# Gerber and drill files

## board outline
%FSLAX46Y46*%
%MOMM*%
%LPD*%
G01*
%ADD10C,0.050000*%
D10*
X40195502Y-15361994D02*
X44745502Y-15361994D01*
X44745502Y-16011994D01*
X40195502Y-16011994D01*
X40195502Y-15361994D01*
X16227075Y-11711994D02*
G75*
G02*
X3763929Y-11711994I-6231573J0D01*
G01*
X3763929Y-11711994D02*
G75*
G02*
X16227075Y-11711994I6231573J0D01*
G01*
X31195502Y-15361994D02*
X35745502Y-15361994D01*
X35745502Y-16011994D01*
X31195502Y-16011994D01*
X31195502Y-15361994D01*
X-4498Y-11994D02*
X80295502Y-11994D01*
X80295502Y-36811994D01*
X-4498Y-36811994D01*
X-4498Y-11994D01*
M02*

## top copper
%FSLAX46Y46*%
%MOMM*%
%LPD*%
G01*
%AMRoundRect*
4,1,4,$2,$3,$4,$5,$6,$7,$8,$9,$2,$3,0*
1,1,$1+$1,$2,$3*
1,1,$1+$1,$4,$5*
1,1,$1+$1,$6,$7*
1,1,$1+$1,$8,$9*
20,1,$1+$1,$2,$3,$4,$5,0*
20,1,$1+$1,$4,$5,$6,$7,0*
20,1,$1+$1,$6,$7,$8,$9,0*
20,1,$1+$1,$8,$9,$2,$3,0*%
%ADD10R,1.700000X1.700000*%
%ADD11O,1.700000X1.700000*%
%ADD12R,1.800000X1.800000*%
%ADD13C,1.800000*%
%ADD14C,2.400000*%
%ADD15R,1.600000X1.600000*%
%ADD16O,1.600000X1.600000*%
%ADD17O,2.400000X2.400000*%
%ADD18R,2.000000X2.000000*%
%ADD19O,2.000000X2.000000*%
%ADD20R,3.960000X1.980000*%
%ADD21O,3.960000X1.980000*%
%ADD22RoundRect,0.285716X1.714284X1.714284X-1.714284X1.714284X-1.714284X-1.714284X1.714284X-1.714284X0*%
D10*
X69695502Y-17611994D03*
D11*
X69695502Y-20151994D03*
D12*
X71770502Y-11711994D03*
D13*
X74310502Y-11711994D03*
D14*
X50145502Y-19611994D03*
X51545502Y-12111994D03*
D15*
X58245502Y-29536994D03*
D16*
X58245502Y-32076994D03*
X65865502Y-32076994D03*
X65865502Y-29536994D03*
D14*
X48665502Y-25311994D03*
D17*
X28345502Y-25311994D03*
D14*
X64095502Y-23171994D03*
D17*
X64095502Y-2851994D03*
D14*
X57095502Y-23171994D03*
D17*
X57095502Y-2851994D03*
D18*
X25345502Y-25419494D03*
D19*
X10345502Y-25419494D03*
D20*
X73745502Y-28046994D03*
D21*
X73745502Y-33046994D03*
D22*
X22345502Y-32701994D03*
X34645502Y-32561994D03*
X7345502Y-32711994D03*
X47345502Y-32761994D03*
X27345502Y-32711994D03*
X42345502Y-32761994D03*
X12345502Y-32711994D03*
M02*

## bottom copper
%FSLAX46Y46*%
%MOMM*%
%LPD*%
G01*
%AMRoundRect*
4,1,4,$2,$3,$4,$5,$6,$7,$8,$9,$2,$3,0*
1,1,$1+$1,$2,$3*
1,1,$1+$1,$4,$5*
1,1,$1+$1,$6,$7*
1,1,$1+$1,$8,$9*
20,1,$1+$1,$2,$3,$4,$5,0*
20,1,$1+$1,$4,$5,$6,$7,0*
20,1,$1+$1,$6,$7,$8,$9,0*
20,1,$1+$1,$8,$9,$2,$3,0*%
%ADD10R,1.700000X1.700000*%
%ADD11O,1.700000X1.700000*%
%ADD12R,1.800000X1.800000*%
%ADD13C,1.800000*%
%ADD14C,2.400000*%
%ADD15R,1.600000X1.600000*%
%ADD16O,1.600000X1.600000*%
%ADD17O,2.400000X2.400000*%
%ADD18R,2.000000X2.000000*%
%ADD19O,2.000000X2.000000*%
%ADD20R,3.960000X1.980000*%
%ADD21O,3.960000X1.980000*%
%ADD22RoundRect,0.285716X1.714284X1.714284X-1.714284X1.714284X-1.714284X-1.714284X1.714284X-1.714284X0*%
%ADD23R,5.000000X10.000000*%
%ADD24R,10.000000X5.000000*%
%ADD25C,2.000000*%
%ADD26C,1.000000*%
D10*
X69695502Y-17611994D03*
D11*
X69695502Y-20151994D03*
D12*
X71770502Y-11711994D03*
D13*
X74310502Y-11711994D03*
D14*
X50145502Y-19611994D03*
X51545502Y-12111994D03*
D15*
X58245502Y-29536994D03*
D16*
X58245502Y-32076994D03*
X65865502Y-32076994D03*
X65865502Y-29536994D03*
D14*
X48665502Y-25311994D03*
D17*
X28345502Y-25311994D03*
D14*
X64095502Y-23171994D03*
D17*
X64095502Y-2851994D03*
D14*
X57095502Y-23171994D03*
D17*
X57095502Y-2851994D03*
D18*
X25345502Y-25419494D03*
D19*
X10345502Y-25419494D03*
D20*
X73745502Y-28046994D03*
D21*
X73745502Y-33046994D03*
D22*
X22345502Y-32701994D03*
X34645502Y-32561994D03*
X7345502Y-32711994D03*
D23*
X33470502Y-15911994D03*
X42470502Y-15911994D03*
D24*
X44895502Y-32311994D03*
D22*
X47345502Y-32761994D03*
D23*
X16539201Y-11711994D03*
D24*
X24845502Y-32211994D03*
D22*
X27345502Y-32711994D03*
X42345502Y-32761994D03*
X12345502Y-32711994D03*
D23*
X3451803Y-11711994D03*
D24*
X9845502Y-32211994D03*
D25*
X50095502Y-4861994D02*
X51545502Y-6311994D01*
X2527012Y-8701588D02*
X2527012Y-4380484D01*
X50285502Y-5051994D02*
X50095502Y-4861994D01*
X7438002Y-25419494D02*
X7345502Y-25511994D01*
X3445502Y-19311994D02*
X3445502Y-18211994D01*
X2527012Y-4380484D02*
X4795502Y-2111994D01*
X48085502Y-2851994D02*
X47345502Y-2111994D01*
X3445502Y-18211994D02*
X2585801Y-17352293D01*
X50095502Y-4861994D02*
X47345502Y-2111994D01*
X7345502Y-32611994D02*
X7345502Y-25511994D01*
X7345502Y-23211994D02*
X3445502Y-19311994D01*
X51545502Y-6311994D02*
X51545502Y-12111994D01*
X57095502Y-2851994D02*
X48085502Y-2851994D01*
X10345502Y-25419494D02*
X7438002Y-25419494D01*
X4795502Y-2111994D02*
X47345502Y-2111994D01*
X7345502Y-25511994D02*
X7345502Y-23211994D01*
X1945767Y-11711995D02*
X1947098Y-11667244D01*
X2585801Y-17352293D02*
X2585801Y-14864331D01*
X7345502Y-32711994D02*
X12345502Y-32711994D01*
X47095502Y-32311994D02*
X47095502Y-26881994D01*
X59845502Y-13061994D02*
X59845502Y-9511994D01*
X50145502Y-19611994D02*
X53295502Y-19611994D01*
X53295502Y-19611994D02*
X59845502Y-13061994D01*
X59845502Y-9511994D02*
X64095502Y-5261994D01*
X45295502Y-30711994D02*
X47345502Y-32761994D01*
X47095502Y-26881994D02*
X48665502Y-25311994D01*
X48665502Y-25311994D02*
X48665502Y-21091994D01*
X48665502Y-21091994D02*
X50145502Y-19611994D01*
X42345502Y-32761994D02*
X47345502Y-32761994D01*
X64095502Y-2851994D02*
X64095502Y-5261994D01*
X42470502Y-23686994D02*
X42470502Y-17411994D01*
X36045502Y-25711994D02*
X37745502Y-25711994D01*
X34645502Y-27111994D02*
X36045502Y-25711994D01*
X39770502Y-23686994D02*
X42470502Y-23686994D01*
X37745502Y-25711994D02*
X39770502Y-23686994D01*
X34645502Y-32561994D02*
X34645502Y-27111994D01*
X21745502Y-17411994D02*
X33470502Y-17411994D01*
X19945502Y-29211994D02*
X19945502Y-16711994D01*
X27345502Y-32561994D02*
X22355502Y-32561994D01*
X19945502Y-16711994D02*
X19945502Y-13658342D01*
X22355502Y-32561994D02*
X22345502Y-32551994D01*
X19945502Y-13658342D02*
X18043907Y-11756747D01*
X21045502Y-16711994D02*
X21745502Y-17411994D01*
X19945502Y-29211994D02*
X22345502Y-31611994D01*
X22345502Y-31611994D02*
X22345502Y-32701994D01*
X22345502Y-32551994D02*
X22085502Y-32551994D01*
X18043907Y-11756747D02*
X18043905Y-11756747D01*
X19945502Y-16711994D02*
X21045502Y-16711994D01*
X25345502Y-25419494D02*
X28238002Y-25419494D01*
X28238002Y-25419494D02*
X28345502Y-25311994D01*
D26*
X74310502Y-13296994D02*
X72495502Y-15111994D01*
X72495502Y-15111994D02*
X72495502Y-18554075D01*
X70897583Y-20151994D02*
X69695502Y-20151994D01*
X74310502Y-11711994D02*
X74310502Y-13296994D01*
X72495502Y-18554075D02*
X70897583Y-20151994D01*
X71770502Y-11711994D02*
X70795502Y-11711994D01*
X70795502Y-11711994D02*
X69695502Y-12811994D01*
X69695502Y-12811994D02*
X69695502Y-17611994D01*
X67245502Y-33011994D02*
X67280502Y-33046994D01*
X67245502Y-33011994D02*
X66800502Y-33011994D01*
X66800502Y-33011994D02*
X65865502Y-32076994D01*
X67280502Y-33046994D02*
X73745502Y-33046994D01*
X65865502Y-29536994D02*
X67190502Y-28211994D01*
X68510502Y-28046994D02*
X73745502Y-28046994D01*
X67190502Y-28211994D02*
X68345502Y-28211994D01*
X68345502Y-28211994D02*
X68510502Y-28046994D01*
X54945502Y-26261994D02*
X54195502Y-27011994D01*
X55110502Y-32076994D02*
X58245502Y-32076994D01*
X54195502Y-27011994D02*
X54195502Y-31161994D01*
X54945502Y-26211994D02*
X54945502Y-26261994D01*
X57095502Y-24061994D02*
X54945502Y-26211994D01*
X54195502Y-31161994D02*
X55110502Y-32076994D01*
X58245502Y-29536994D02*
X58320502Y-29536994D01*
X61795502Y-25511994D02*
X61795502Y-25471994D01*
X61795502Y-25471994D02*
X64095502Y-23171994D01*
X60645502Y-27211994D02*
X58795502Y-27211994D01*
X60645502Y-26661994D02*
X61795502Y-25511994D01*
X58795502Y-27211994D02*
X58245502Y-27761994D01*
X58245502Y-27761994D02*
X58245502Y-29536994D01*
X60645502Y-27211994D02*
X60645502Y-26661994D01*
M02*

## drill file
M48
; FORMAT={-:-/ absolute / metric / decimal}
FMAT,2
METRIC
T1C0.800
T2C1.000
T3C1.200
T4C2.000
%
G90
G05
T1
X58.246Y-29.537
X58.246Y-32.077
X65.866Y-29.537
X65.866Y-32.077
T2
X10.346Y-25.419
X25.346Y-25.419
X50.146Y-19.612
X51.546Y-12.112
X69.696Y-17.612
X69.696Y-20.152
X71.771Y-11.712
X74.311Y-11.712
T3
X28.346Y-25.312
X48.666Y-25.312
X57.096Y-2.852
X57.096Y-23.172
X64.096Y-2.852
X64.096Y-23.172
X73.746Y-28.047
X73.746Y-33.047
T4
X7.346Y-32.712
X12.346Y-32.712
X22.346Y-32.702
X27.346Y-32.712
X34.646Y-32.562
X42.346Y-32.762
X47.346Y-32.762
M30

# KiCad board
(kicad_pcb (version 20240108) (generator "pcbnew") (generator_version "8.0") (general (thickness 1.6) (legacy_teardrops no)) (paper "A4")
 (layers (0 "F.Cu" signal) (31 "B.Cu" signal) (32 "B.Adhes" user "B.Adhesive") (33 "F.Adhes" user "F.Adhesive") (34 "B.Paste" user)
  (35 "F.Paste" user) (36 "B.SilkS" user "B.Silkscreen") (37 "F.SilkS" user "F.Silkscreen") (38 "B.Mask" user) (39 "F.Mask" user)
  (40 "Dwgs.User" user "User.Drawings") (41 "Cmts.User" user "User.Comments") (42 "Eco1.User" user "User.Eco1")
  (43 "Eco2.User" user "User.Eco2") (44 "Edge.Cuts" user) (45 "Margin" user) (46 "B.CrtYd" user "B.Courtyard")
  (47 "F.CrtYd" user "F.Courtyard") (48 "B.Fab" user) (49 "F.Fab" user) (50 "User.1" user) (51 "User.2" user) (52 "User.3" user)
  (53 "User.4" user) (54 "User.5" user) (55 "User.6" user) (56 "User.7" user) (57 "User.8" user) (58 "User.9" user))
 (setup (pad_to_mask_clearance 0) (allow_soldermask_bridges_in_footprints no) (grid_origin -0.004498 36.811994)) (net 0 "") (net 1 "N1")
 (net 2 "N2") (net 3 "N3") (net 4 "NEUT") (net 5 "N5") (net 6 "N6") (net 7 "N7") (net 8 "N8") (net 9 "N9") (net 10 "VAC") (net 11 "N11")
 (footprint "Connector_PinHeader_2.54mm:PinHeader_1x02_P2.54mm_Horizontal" (layer "F.Cu") (at 69.695502 17.611994)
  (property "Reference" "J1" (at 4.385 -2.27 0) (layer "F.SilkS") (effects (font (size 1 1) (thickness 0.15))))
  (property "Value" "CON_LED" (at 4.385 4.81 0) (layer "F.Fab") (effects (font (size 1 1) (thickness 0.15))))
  (pad "1" thru_hole rect (at 0 0) (size 1.7 1.7) (drill 1) (layers "*.Cu" "*.Mask") (remove_unused_layers no) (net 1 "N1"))
  (pad "2" thru_hole oval (at 0 2.54) (size 1.7 1.7) (drill 1) (layers "*.Cu" "*.Mask") (remove_unused_layers no) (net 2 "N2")))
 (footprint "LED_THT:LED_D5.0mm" (layer "F.Cu") (at 71.770502 11.711994)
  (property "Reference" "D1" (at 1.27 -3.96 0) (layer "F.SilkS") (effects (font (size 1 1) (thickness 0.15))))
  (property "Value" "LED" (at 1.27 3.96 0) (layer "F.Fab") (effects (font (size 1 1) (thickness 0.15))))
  (pad "1" thru_hole rect (at 0 0) (size 1.8 1.8) (drill 1) (layers "*.Cu" "*.Mask") (remove_unused_layers no) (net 1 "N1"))
  (pad "2" thru_hole circle (at 2.54 0) (size 1.8 1.8) (drill 1) (layers "*.Cu" "*.Mask") (remove_unused_layers no) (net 2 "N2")))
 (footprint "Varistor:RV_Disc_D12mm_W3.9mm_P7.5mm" (layer "F.Cu") (at 50.145502 19.611994 90)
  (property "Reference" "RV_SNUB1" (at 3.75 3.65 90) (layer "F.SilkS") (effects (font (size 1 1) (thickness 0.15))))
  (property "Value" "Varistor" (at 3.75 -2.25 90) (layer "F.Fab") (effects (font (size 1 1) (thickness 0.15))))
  (pad "1" thru_hole circle (at 0 0 90) (size 2.4 2.4) (drill 1) (layers "*.Cu" "*.Mask") (remove_unused_layers no) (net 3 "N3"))
  (pad "2" thru_hole circle (at 7.5 1.4 90) (size 2.4 2.4) (drill 1) (layers "*.Cu" "*.Mask") (remove_unused_layers no) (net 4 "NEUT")))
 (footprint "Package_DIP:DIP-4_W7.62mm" (layer "F.Cu") (at 58.245502 29.536994)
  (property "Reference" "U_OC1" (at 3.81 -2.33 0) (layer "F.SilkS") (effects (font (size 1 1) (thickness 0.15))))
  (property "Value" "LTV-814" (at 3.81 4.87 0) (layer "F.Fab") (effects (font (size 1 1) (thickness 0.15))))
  (pad "1" thru_hole rect (at 0 0) (size 1.6 1.6) (drill 0.8) (layers "*.Cu" "*.Mask") (remove_unused_layers no) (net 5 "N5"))
  (pad "2" thru_hole oval (at 0 2.54) (size 1.6 1.6) (drill 0.8) (layers "*.Cu" "*.Mask") (remove_unused_layers no) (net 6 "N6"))
  (pad "3" thru_hole oval (at 7.62 2.54) (size 1.6 1.6) (drill 0.8) (layers "*.Cu" "*.Mask") (remove_unused_layers no) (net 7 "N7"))
  (pad "4" thru_hole oval (at 7.62 0) (size 1.6 1.6) (drill 0.8) (layers "*.Cu" "*.Mask") (remove_unused_layers no) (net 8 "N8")))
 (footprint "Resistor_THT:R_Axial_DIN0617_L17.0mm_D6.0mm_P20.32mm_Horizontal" (layer "F.Cu") (at 48.665502 25.311994 180)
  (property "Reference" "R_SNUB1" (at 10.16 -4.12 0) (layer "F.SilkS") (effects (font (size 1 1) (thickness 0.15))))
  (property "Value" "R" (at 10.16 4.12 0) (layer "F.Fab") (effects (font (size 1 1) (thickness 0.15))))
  (pad "1" thru_hole circle (at 0 0 180) (size 2.4 2.4) (drill 1.2) (layers "*.Cu" "*.Mask") (remove_unused_layers no) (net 3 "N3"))
  (pad "2" thru_hole oval (at 20.32 0 180) (size 2.4 2.4) (drill 1.2) (layers "*.Cu" "*.Mask") (remove_unused_layers no) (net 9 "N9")))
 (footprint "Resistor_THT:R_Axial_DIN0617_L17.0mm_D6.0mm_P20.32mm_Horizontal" (layer "F.Cu") (at 64.095502 23.171994 90)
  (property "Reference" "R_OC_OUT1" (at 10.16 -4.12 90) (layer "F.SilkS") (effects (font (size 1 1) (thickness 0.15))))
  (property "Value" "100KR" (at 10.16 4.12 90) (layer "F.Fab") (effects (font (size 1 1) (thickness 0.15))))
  (pad "1" thru_hole circle (at 0 0 90) (size 2.4 2.4) (drill 1.2) (layers "*.Cu" "*.Mask") (remove_unused_layers no) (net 5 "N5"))
  (pad "2" thru_hole oval (at 20.32 0 90) (size 2.4 2.4) (drill 1.2) (layers "*.Cu" "*.Mask") (remove_unused_layers no) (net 3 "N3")))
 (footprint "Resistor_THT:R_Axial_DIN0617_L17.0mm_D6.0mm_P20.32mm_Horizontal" (layer "F.Cu") (at 57.095502 23.171994 90)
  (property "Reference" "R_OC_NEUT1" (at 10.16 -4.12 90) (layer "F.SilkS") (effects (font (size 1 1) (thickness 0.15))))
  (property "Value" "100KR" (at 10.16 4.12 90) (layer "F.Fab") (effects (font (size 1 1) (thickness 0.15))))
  (pad "1" thru_hole circle (at 0 0 90) (size 2.4 2.4) (drill 1.2) (layers "*.Cu" "*.Mask") (remove_unused_layers no) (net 6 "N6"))
  (pad "2" thru_hole oval (at 20.32 0 90) (size 2.4 2.4) (drill 1.2) (layers "*.Cu" "*.Mask") (remove_unused_layers no) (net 4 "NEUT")))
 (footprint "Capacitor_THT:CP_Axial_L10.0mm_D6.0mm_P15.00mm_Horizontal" (layer "F.Cu") (at 25.345502 25.419494 180)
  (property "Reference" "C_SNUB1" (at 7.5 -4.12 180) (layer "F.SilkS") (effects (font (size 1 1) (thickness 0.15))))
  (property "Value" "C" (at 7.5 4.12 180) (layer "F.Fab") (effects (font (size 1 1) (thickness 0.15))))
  (pad "1" thru_hole rect (at 0 0 180) (size 2 2) (drill 1) (layers "*.Cu" "*.Mask") (remove_unused_layers no) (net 9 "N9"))
  (pad "2" thru_hole oval (at 15 0 180) (size 2 2) (drill 1) (layers "*.Cu" "*.Mask") (remove_unused_layers no) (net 4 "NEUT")))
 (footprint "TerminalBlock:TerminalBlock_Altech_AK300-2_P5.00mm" (layer "F.Cu") (at 73.745502 28.046994 -90)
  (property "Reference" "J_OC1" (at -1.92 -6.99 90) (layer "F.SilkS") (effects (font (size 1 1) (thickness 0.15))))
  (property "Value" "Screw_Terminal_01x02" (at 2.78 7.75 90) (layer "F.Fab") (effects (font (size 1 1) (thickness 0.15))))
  (pad "1" thru_hole rect (at 0 0 270) (size 1.98 3.96) (drill 1.2) (layers "*.Cu" "*.Mask") (remove_unused_layers no) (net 8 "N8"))
  (pad "2" thru_hole oval (at 5 0 270) (size 1.98 3.96) (drill 1.2) (layers "*.Cu" "*.Mask") (remove_unused_layers no) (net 7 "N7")))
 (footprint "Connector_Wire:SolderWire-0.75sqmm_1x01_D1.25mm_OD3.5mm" (layer "B.Cu") (at 22.345502 32.701994 180)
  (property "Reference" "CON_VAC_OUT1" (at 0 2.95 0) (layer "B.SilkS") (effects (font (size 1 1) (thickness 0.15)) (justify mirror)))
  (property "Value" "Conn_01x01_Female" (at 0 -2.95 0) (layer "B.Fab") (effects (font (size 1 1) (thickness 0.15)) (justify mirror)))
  (pad "1" thru_hole roundrect (at 0 0 180) (size 4 4) (drill 2) (layers "*.Cu" "*.Mask") (remove_unused_layers no)
   (roundrect_rratio 0.071429) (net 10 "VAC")))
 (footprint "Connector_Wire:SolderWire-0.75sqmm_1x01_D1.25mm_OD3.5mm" (layer "B.Cu") (at 34.645502 32.561994 180)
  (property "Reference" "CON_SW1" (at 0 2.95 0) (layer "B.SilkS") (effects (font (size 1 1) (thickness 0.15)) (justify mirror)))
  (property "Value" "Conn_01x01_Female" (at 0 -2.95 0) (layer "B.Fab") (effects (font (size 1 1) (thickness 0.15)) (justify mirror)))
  (pad "1" thru_hole roundrect (at 0 0 180) (size 4 4) (drill 2) (layers "*.Cu" "*.Mask") (remove_unused_layers no)
   (roundrect_rratio 0.071429) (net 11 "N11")))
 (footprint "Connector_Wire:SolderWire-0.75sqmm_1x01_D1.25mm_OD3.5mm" (layer "B.Cu") (at 7.345502 32.711994 180)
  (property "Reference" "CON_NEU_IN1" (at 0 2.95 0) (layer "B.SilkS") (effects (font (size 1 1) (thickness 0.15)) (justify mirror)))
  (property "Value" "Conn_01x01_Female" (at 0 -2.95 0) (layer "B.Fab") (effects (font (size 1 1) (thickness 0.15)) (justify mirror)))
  (pad "1" thru_hole roundrect (at 0 0 180) (size 4 4) (drill 2) (layers "*.Cu" "*.Mask") (remove_unused_layers no)
   (roundrect_rratio 0.071429) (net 4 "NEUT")))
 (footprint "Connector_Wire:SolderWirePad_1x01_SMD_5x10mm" (layer "B.Cu") (at 33.470502 15.911994 180)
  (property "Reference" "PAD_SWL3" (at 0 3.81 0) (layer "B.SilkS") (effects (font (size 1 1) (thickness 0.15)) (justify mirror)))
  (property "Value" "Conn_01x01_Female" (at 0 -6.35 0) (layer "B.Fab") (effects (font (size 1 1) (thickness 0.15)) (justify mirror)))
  (pad "1" smd rect (at 0 0 180) (size 5 10) (layers "B.Cu" "B.Paste" "B.Mask") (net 10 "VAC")))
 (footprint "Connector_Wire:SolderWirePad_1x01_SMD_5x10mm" (layer "B.Cu") (at 42.470502 15.911994 180)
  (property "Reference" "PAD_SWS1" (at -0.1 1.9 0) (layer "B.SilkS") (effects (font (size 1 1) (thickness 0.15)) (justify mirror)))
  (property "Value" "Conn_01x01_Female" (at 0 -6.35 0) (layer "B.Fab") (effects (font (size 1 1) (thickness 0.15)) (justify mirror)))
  (pad "1" smd rect (at 0 0 180) (size 5 10) (layers "B.Cu" "B.Paste" "B.Mask") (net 11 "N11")))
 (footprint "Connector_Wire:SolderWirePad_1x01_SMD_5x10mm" (layer "B.Cu") (at 44.895502 32.311994 -90)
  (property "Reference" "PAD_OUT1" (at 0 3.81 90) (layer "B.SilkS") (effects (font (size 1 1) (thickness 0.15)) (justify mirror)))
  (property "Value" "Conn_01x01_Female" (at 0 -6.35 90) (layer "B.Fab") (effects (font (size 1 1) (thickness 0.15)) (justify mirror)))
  (pad "1" smd rect (at 0 0 270) (size 5 10) (layers "B.Cu" "B.Paste" "B.Mask") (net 3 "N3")))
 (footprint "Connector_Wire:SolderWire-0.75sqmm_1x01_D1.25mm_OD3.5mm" (layer "B.Cu") (at 47.345502 32.761994 180)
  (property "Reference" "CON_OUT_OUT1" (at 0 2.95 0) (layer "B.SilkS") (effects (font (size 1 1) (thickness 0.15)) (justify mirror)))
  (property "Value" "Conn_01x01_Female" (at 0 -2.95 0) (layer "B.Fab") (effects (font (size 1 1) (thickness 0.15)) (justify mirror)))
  (pad "1" thru_hole roundrect (at 0 0 180) (size 4 4) (drill 2) (layers "*.Cu" "*.Mask") (remove_unused_layers no)
   (roundrect_rratio 0.071429) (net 3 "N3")))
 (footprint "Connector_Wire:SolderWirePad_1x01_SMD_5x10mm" (layer "B.Cu") (at 16.539201 11.711994 180)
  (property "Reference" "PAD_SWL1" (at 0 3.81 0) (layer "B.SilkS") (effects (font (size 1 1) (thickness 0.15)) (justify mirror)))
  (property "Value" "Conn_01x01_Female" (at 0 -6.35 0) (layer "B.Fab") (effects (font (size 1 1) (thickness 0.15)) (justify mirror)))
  (pad "1" smd rect (at 0 0 180) (size 5 10) (layers "B.Cu" "B.Paste" "B.Mask") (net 10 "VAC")))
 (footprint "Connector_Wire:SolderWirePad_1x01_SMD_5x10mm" (layer "B.Cu") (at 24.845502 32.211994 -90)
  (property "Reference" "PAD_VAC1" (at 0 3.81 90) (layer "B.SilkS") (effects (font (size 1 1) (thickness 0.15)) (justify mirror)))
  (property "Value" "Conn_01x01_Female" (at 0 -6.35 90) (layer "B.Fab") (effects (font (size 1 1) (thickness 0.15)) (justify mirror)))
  (pad "1" smd rect (at 0 0 270) (size 5 10) (layers "B.Cu" "B.Paste" "B.Mask") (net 10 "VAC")))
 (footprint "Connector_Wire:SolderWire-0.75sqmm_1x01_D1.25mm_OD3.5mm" (layer "B.Cu") (at 27.345502 32.711994 180)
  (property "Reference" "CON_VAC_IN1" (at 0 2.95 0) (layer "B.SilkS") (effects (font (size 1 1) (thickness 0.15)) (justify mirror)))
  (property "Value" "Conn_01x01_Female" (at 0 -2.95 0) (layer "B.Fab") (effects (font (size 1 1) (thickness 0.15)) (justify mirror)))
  (pad "1" thru_hole roundrect (at 0 0 180) (size 4 4) (drill 2) (layers "*.Cu" "*.Mask") (remove_unused_layers no)
   (roundrect_rratio 0.071429) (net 10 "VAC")))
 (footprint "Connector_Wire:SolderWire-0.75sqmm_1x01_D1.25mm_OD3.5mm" (layer "B.Cu") (at 42.345502 32.761994 180)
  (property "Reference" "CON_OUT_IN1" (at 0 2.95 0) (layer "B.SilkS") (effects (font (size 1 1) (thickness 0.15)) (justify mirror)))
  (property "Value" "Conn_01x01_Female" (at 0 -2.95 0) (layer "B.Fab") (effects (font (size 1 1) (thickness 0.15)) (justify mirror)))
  (pad "1" thru_hole roundrect (at 0 0 180) (size 4 4) (drill 2) (layers "*.Cu" "*.Mask") (remove_unused_layers no)
   (roundrect_rratio 0.071429) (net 3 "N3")))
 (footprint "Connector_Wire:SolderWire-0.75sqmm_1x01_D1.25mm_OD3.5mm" (layer "B.Cu") (at 12.345502 32.711994 180)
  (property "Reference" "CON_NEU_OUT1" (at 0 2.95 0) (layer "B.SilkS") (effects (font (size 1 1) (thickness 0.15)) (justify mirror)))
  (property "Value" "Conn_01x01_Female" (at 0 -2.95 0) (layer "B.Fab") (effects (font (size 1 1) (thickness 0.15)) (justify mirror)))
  (pad "1" thru_hole roundrect (at 0 0 180) (size 4 4) (drill 2) (layers "*.Cu" "*.Mask") (remove_unused_layers no)
   (roundrect_rratio 0.071429) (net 4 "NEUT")))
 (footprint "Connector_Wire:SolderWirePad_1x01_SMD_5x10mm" (layer "B.Cu") (at 3.451803 11.711994 180)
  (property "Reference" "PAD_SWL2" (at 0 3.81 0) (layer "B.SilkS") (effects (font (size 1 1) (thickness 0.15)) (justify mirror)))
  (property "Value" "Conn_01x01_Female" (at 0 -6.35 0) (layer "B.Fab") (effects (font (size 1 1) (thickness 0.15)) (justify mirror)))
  (pad "1" smd rect (at 0 0 180) (size 5 10) (layers "B.Cu" "B.Paste" "B.Mask") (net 4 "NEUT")))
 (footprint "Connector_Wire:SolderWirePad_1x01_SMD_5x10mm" (layer "B.Cu") (at 9.845502 32.211994 -90)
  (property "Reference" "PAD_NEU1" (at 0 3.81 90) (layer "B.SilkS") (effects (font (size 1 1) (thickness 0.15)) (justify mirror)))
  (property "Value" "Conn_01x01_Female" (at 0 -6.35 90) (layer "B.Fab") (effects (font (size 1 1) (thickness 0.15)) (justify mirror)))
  (pad "1" smd rect (at 0 0 270) (size 5 10) (layers "B.Cu" "B.Paste" "B.Mask") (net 4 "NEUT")))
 (gr_rect (start 40.195502 15.361994) (end 44.745502 16.011994) (stroke (width 0.05) (type default)) (fill none) (layer "Edge.Cuts"))
 (gr_circle (center 9.995502 11.711994) (end 13.845502 16.611994) (stroke (width 0.05) (type default)) (fill none) (layer "Edge.Cuts"))
 (gr_rect (start 31.195502 15.361994) (end 35.745502 16.011994) (stroke (width 0.05) (type default)) (fill none) (layer "Edge.Cuts"))
 (gr_rect (start -0.004498 0.011994) (end 80.295502 36.811994) (stroke (width 0.05) (type default)) (fill none) (layer "Edge.Cuts"))
 (segment (start 50.095502 4.861994) (end 51.545502 6.311994) (width 2) (layer "B.Cu") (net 4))
 (segment (start 2.527012 8.701588) (end 2.527012 4.380484) (width 2) (layer "B.Cu") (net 4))
 (segment (start 50.285502 5.051994) (end 50.095502 4.861994) (width 2) (layer "B.Cu") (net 4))
 (segment (start 7.438002 25.419494) (end 7.345502 25.511994) (width 2) (layer "B.Cu") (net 4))
 (segment (start 3.445502 19.311994) (end 3.445502 18.211994) (width 2) (layer "B.Cu") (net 4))
 (segment (start 2.527012 4.380484) (end 4.795502 2.111994) (width 2) (layer "B.Cu") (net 4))
 (segment (start 48.085502 2.851994) (end 47.345502 2.111994) (width 2) (layer "B.Cu") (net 4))
 (segment (start 3.445502 18.211994) (end 2.585801 17.352293) (width 2) (layer "B.Cu") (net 4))
 (segment (start 50.095502 4.861994) (end 47.345502 2.111994) (width 2) (layer "B.Cu") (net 4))
 (segment (start 7.345502 32.611994) (end 7.345502 25.511994) (width 2) (layer "B.Cu") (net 4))
 (segment (start 7.345502 23.211994) (end 3.445502 19.311994) (width 2) (layer "B.Cu") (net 4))
 (segment (start 51.545502 6.311994) (end 51.545502 12.111994) (width 2) (layer "B.Cu") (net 4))
 (segment (start 57.095502 2.851994) (end 48.085502 2.851994) (width 2) (layer "B.Cu") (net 4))
 (segment (start 10.345502 25.419494) (end 7.438002 25.419494) (width 2) (layer "B.Cu") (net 4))
 (segment (start 4.795502 2.111994) (end 47.345502 2.111994) (width 2) (layer "B.Cu") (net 4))
 (segment (start 7.345502 25.511994) (end 7.345502 23.211994) (width 2) (layer "B.Cu") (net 4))
 (segment (start 1.945767 11.711995) (end 1.947098 11.667244) (width 2) (layer "B.Cu") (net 4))
 (segment (start 2.585801 17.352293) (end 2.585801 14.864331) (width 2) (layer "B.Cu") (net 4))
 (segment (start 7.345502 32.711994) (end 12.345502 32.711994) (width 2) (layer "B.Cu") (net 4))
 (segment (start 47.095502 32.311994) (end 47.095502 26.881994) (width 2) (layer "B.Cu") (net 3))
 (segment (start 59.845502 13.061994) (end 59.845502 9.511994) (width 2) (layer "B.Cu") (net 3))
 (segment (start 50.145502 19.611994) (end 53.295502 19.611994) (width 2) (layer "B.Cu") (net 3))
 (segment (start 53.295502 19.611994) (end 59.845502 13.061994) (width 2) (layer "B.Cu") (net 3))
 (segment (start 59.845502 9.511994) (end 64.095502 5.261994) (width 2) (layer "B.Cu") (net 3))
 (segment (start 45.295502 30.711994) (end 47.345502 32.761994) (width 2) (layer "B.Cu") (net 3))
 (segment (start 47.095502 26.881994) (end 48.665502 25.311994) (width 2) (layer "B.Cu") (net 3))
 (segment (start 48.665502 25.311994) (end 48.665502 21.091994) (width 2) (layer "B.Cu") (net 3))
 (segment (start 48.665502 21.091994) (end 50.145502 19.611994) (width 2) (layer "B.Cu") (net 3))
 (segment (start 42.345502 32.761994) (end 47.345502 32.761994) (width 2) (layer "B.Cu") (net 3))
 (segment (start 64.095502 2.851994) (end 64.095502 5.261994) (width 2) (layer "B.Cu") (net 3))
 (segment (start 42.470502 23.686994) (end 42.470502 17.411994) (width 2) (layer "B.Cu") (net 11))
 (segment (start 36.045502 25.711994) (end 37.745502 25.711994) (width 2) (layer "B.Cu") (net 11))
 (segment (start 34.645502 27.111994) (end 36.045502 25.711994) (width 2) (layer "B.Cu") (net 11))
 (segment (start 39.770502 23.686994) (end 42.470502 23.686994) (width 2) (layer "B.Cu") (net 11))
 (segment (start 37.745502 25.711994) (end 39.770502 23.686994) (width 2) (layer "B.Cu") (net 11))
 (segment (start 34.645502 32.561994) (end 34.645502 27.111994) (width 2) (layer "B.Cu") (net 11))
 (segment (start 21.745502 17.411994) (end 33.470502 17.411994) (width 2) (layer "B.Cu") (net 10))
 (segment (start 19.945502 29.211994) (end 19.945502 16.711994) (width 2) (layer "B.Cu") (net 10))
 (segment (start 27.345502 32.561994) (end 22.355502 32.561994) (width 2) (layer "B.Cu") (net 10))
 (segment (start 19.945502 16.711994) (end 19.945502 13.658342) (width 2) (layer "B.Cu") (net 10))
 (segment (start 22.355502 32.561994) (end 22.345502 32.551994) (width 2) (layer "B.Cu") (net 10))
 (segment (start 19.945502 13.658342) (end 18.043907 11.756747) (width 2) (layer "B.Cu") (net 10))
 (segment (start 21.045502 16.711994) (end 21.745502 17.411994) (width 2) (layer "B.Cu") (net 10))
 (segment (start 19.945502 29.211994) (end 22.345502 31.611994) (width 2) (layer "B.Cu") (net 10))
 (segment (start 22.345502 31.611994) (end 22.345502 32.701994) (width 2) (layer "B.Cu") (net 10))
 (segment (start 22.345502 32.551994) (end 22.085502 32.551994) (width 2) (layer "B.Cu") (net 10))
 (segment (start 18.043907 11.756747) (end 18.043905 11.756747) (width 2) (layer "B.Cu") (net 10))
 (segment (start 19.945502 16.711994) (end 21.045502 16.711994) (width 2) (layer "B.Cu") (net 10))
 (segment (start 25.345502 25.419494) (end 28.238002 25.419494) (width 2) (layer "B.Cu") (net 9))
 (segment (start 28.238002 25.419494) (end 28.345502 25.311994) (width 2) (layer "B.Cu") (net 9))
 (segment (start 74.310502 13.296994) (end 72.495502 15.111994) (width 1) (layer "B.Cu") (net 2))
 (segment (start 72.495502 15.111994) (end 72.495502 18.554075) (width 1) (layer "B.Cu") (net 2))
 (segment (start 70.897583 20.151994) (end 69.695502 20.151994) (width 1) (layer "B.Cu") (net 2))
 (segment (start 74.310502 11.711994) (end 74.310502 13.296994) (width 1) (layer "B.Cu") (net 2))
 (segment (start 72.495502 18.554075) (end 70.897583 20.151994) (width 1) (layer "B.Cu") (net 2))
 (segment (start 71.770502 11.711994) (end 70.795502 11.711994) (width 1) (layer "B.Cu") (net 1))
 (segment (start 70.795502 11.711994) (end 69.695502 12.811994) (width 1) (layer "B.Cu") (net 1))
 (segment (start 69.695502 12.811994) (end 69.695502 17.611994) (width 1) (layer "B.Cu") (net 1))
 (segment (start 67.245502 33.011994) (end 67.280502 33.046994) (width 1) (layer "B.Cu") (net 7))
 (segment (start 67.245502 33.011994) (end 66.800502 33.011994) (width 1) (layer "B.Cu") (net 7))
 (segment (start 66.800502 33.011994) (end 65.865502 32.076994) (width 1) (layer "B.Cu") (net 7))
 (segment (start 67.280502 33.046994) (end 73.745502 33.046994) (width 1) (layer "B.Cu") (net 7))
 (segment (start 65.865502 29.536994) (end 67.190502 28.211994) (width 1) (layer "B.Cu") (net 8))
 (segment (start 68.510502 28.046994) (end 73.745502 28.046994) (width 1) (layer "B.Cu") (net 8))
 (segment (start 67.190502 28.211994) (end 68.345502 28.211994) (width 1) (layer "B.Cu") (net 8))
 (segment (start 68.345502 28.211994) (end 68.510502 28.046994) (width 1) (layer "B.Cu") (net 8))
 (segment (start 54.945502 26.261994) (end 54.195502 27.011994) (width 1) (layer "B.Cu") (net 6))
 (segment (start 55.110502 32.076994) (end 58.245502 32.076994) (width 1) (layer "B.Cu") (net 6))
 (segment (start 54.195502 27.011994) (end 54.195502 31.161994) (width 1) (layer "B.Cu") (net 6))
 (segment (start 54.945502 26.211994) (end 54.945502 26.261994) (width 1) (layer "B.Cu") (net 6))
 (segment (start 57.095502 24.061994) (end 54.945502 26.211994) (width 1) (layer "B.Cu") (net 6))
 (segment (start 54.195502 31.161994) (end 55.110502 32.076994) (width 1) (layer "B.Cu") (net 6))
 (segment (start 58.245502 29.536994) (end 58.320502 29.536994) (width 1) (layer "B.Cu") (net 5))
 (segment (start 61.795502 25.511994) (end 61.795502 25.471994) (width 1) (layer "B.Cu") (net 5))
 (segment (start 61.795502 25.471994) (end 64.095502 23.171994) (width 1) (layer "B.Cu") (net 5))
 (segment (start 60.645502 27.211994) (end 58.795502 27.211994) (width 1) (layer "B.Cu") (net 5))
 (segment (start 60.645502 26.661994) (end 61.795502 25.511994) (width 1) (layer "B.Cu") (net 5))
 (segment (start 58.795502 27.211994) (end 58.245502 27.761994) (width 1) (layer "B.Cu") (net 5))
 (segment (start 58.245502 27.761994) (end 58.245502 29.536994) (width 1) (layer "B.Cu") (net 5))
 (segment (start 60.645502 27.211994) (end 60.645502 26.661994) (width 1) (layer "B.Cu") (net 5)))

